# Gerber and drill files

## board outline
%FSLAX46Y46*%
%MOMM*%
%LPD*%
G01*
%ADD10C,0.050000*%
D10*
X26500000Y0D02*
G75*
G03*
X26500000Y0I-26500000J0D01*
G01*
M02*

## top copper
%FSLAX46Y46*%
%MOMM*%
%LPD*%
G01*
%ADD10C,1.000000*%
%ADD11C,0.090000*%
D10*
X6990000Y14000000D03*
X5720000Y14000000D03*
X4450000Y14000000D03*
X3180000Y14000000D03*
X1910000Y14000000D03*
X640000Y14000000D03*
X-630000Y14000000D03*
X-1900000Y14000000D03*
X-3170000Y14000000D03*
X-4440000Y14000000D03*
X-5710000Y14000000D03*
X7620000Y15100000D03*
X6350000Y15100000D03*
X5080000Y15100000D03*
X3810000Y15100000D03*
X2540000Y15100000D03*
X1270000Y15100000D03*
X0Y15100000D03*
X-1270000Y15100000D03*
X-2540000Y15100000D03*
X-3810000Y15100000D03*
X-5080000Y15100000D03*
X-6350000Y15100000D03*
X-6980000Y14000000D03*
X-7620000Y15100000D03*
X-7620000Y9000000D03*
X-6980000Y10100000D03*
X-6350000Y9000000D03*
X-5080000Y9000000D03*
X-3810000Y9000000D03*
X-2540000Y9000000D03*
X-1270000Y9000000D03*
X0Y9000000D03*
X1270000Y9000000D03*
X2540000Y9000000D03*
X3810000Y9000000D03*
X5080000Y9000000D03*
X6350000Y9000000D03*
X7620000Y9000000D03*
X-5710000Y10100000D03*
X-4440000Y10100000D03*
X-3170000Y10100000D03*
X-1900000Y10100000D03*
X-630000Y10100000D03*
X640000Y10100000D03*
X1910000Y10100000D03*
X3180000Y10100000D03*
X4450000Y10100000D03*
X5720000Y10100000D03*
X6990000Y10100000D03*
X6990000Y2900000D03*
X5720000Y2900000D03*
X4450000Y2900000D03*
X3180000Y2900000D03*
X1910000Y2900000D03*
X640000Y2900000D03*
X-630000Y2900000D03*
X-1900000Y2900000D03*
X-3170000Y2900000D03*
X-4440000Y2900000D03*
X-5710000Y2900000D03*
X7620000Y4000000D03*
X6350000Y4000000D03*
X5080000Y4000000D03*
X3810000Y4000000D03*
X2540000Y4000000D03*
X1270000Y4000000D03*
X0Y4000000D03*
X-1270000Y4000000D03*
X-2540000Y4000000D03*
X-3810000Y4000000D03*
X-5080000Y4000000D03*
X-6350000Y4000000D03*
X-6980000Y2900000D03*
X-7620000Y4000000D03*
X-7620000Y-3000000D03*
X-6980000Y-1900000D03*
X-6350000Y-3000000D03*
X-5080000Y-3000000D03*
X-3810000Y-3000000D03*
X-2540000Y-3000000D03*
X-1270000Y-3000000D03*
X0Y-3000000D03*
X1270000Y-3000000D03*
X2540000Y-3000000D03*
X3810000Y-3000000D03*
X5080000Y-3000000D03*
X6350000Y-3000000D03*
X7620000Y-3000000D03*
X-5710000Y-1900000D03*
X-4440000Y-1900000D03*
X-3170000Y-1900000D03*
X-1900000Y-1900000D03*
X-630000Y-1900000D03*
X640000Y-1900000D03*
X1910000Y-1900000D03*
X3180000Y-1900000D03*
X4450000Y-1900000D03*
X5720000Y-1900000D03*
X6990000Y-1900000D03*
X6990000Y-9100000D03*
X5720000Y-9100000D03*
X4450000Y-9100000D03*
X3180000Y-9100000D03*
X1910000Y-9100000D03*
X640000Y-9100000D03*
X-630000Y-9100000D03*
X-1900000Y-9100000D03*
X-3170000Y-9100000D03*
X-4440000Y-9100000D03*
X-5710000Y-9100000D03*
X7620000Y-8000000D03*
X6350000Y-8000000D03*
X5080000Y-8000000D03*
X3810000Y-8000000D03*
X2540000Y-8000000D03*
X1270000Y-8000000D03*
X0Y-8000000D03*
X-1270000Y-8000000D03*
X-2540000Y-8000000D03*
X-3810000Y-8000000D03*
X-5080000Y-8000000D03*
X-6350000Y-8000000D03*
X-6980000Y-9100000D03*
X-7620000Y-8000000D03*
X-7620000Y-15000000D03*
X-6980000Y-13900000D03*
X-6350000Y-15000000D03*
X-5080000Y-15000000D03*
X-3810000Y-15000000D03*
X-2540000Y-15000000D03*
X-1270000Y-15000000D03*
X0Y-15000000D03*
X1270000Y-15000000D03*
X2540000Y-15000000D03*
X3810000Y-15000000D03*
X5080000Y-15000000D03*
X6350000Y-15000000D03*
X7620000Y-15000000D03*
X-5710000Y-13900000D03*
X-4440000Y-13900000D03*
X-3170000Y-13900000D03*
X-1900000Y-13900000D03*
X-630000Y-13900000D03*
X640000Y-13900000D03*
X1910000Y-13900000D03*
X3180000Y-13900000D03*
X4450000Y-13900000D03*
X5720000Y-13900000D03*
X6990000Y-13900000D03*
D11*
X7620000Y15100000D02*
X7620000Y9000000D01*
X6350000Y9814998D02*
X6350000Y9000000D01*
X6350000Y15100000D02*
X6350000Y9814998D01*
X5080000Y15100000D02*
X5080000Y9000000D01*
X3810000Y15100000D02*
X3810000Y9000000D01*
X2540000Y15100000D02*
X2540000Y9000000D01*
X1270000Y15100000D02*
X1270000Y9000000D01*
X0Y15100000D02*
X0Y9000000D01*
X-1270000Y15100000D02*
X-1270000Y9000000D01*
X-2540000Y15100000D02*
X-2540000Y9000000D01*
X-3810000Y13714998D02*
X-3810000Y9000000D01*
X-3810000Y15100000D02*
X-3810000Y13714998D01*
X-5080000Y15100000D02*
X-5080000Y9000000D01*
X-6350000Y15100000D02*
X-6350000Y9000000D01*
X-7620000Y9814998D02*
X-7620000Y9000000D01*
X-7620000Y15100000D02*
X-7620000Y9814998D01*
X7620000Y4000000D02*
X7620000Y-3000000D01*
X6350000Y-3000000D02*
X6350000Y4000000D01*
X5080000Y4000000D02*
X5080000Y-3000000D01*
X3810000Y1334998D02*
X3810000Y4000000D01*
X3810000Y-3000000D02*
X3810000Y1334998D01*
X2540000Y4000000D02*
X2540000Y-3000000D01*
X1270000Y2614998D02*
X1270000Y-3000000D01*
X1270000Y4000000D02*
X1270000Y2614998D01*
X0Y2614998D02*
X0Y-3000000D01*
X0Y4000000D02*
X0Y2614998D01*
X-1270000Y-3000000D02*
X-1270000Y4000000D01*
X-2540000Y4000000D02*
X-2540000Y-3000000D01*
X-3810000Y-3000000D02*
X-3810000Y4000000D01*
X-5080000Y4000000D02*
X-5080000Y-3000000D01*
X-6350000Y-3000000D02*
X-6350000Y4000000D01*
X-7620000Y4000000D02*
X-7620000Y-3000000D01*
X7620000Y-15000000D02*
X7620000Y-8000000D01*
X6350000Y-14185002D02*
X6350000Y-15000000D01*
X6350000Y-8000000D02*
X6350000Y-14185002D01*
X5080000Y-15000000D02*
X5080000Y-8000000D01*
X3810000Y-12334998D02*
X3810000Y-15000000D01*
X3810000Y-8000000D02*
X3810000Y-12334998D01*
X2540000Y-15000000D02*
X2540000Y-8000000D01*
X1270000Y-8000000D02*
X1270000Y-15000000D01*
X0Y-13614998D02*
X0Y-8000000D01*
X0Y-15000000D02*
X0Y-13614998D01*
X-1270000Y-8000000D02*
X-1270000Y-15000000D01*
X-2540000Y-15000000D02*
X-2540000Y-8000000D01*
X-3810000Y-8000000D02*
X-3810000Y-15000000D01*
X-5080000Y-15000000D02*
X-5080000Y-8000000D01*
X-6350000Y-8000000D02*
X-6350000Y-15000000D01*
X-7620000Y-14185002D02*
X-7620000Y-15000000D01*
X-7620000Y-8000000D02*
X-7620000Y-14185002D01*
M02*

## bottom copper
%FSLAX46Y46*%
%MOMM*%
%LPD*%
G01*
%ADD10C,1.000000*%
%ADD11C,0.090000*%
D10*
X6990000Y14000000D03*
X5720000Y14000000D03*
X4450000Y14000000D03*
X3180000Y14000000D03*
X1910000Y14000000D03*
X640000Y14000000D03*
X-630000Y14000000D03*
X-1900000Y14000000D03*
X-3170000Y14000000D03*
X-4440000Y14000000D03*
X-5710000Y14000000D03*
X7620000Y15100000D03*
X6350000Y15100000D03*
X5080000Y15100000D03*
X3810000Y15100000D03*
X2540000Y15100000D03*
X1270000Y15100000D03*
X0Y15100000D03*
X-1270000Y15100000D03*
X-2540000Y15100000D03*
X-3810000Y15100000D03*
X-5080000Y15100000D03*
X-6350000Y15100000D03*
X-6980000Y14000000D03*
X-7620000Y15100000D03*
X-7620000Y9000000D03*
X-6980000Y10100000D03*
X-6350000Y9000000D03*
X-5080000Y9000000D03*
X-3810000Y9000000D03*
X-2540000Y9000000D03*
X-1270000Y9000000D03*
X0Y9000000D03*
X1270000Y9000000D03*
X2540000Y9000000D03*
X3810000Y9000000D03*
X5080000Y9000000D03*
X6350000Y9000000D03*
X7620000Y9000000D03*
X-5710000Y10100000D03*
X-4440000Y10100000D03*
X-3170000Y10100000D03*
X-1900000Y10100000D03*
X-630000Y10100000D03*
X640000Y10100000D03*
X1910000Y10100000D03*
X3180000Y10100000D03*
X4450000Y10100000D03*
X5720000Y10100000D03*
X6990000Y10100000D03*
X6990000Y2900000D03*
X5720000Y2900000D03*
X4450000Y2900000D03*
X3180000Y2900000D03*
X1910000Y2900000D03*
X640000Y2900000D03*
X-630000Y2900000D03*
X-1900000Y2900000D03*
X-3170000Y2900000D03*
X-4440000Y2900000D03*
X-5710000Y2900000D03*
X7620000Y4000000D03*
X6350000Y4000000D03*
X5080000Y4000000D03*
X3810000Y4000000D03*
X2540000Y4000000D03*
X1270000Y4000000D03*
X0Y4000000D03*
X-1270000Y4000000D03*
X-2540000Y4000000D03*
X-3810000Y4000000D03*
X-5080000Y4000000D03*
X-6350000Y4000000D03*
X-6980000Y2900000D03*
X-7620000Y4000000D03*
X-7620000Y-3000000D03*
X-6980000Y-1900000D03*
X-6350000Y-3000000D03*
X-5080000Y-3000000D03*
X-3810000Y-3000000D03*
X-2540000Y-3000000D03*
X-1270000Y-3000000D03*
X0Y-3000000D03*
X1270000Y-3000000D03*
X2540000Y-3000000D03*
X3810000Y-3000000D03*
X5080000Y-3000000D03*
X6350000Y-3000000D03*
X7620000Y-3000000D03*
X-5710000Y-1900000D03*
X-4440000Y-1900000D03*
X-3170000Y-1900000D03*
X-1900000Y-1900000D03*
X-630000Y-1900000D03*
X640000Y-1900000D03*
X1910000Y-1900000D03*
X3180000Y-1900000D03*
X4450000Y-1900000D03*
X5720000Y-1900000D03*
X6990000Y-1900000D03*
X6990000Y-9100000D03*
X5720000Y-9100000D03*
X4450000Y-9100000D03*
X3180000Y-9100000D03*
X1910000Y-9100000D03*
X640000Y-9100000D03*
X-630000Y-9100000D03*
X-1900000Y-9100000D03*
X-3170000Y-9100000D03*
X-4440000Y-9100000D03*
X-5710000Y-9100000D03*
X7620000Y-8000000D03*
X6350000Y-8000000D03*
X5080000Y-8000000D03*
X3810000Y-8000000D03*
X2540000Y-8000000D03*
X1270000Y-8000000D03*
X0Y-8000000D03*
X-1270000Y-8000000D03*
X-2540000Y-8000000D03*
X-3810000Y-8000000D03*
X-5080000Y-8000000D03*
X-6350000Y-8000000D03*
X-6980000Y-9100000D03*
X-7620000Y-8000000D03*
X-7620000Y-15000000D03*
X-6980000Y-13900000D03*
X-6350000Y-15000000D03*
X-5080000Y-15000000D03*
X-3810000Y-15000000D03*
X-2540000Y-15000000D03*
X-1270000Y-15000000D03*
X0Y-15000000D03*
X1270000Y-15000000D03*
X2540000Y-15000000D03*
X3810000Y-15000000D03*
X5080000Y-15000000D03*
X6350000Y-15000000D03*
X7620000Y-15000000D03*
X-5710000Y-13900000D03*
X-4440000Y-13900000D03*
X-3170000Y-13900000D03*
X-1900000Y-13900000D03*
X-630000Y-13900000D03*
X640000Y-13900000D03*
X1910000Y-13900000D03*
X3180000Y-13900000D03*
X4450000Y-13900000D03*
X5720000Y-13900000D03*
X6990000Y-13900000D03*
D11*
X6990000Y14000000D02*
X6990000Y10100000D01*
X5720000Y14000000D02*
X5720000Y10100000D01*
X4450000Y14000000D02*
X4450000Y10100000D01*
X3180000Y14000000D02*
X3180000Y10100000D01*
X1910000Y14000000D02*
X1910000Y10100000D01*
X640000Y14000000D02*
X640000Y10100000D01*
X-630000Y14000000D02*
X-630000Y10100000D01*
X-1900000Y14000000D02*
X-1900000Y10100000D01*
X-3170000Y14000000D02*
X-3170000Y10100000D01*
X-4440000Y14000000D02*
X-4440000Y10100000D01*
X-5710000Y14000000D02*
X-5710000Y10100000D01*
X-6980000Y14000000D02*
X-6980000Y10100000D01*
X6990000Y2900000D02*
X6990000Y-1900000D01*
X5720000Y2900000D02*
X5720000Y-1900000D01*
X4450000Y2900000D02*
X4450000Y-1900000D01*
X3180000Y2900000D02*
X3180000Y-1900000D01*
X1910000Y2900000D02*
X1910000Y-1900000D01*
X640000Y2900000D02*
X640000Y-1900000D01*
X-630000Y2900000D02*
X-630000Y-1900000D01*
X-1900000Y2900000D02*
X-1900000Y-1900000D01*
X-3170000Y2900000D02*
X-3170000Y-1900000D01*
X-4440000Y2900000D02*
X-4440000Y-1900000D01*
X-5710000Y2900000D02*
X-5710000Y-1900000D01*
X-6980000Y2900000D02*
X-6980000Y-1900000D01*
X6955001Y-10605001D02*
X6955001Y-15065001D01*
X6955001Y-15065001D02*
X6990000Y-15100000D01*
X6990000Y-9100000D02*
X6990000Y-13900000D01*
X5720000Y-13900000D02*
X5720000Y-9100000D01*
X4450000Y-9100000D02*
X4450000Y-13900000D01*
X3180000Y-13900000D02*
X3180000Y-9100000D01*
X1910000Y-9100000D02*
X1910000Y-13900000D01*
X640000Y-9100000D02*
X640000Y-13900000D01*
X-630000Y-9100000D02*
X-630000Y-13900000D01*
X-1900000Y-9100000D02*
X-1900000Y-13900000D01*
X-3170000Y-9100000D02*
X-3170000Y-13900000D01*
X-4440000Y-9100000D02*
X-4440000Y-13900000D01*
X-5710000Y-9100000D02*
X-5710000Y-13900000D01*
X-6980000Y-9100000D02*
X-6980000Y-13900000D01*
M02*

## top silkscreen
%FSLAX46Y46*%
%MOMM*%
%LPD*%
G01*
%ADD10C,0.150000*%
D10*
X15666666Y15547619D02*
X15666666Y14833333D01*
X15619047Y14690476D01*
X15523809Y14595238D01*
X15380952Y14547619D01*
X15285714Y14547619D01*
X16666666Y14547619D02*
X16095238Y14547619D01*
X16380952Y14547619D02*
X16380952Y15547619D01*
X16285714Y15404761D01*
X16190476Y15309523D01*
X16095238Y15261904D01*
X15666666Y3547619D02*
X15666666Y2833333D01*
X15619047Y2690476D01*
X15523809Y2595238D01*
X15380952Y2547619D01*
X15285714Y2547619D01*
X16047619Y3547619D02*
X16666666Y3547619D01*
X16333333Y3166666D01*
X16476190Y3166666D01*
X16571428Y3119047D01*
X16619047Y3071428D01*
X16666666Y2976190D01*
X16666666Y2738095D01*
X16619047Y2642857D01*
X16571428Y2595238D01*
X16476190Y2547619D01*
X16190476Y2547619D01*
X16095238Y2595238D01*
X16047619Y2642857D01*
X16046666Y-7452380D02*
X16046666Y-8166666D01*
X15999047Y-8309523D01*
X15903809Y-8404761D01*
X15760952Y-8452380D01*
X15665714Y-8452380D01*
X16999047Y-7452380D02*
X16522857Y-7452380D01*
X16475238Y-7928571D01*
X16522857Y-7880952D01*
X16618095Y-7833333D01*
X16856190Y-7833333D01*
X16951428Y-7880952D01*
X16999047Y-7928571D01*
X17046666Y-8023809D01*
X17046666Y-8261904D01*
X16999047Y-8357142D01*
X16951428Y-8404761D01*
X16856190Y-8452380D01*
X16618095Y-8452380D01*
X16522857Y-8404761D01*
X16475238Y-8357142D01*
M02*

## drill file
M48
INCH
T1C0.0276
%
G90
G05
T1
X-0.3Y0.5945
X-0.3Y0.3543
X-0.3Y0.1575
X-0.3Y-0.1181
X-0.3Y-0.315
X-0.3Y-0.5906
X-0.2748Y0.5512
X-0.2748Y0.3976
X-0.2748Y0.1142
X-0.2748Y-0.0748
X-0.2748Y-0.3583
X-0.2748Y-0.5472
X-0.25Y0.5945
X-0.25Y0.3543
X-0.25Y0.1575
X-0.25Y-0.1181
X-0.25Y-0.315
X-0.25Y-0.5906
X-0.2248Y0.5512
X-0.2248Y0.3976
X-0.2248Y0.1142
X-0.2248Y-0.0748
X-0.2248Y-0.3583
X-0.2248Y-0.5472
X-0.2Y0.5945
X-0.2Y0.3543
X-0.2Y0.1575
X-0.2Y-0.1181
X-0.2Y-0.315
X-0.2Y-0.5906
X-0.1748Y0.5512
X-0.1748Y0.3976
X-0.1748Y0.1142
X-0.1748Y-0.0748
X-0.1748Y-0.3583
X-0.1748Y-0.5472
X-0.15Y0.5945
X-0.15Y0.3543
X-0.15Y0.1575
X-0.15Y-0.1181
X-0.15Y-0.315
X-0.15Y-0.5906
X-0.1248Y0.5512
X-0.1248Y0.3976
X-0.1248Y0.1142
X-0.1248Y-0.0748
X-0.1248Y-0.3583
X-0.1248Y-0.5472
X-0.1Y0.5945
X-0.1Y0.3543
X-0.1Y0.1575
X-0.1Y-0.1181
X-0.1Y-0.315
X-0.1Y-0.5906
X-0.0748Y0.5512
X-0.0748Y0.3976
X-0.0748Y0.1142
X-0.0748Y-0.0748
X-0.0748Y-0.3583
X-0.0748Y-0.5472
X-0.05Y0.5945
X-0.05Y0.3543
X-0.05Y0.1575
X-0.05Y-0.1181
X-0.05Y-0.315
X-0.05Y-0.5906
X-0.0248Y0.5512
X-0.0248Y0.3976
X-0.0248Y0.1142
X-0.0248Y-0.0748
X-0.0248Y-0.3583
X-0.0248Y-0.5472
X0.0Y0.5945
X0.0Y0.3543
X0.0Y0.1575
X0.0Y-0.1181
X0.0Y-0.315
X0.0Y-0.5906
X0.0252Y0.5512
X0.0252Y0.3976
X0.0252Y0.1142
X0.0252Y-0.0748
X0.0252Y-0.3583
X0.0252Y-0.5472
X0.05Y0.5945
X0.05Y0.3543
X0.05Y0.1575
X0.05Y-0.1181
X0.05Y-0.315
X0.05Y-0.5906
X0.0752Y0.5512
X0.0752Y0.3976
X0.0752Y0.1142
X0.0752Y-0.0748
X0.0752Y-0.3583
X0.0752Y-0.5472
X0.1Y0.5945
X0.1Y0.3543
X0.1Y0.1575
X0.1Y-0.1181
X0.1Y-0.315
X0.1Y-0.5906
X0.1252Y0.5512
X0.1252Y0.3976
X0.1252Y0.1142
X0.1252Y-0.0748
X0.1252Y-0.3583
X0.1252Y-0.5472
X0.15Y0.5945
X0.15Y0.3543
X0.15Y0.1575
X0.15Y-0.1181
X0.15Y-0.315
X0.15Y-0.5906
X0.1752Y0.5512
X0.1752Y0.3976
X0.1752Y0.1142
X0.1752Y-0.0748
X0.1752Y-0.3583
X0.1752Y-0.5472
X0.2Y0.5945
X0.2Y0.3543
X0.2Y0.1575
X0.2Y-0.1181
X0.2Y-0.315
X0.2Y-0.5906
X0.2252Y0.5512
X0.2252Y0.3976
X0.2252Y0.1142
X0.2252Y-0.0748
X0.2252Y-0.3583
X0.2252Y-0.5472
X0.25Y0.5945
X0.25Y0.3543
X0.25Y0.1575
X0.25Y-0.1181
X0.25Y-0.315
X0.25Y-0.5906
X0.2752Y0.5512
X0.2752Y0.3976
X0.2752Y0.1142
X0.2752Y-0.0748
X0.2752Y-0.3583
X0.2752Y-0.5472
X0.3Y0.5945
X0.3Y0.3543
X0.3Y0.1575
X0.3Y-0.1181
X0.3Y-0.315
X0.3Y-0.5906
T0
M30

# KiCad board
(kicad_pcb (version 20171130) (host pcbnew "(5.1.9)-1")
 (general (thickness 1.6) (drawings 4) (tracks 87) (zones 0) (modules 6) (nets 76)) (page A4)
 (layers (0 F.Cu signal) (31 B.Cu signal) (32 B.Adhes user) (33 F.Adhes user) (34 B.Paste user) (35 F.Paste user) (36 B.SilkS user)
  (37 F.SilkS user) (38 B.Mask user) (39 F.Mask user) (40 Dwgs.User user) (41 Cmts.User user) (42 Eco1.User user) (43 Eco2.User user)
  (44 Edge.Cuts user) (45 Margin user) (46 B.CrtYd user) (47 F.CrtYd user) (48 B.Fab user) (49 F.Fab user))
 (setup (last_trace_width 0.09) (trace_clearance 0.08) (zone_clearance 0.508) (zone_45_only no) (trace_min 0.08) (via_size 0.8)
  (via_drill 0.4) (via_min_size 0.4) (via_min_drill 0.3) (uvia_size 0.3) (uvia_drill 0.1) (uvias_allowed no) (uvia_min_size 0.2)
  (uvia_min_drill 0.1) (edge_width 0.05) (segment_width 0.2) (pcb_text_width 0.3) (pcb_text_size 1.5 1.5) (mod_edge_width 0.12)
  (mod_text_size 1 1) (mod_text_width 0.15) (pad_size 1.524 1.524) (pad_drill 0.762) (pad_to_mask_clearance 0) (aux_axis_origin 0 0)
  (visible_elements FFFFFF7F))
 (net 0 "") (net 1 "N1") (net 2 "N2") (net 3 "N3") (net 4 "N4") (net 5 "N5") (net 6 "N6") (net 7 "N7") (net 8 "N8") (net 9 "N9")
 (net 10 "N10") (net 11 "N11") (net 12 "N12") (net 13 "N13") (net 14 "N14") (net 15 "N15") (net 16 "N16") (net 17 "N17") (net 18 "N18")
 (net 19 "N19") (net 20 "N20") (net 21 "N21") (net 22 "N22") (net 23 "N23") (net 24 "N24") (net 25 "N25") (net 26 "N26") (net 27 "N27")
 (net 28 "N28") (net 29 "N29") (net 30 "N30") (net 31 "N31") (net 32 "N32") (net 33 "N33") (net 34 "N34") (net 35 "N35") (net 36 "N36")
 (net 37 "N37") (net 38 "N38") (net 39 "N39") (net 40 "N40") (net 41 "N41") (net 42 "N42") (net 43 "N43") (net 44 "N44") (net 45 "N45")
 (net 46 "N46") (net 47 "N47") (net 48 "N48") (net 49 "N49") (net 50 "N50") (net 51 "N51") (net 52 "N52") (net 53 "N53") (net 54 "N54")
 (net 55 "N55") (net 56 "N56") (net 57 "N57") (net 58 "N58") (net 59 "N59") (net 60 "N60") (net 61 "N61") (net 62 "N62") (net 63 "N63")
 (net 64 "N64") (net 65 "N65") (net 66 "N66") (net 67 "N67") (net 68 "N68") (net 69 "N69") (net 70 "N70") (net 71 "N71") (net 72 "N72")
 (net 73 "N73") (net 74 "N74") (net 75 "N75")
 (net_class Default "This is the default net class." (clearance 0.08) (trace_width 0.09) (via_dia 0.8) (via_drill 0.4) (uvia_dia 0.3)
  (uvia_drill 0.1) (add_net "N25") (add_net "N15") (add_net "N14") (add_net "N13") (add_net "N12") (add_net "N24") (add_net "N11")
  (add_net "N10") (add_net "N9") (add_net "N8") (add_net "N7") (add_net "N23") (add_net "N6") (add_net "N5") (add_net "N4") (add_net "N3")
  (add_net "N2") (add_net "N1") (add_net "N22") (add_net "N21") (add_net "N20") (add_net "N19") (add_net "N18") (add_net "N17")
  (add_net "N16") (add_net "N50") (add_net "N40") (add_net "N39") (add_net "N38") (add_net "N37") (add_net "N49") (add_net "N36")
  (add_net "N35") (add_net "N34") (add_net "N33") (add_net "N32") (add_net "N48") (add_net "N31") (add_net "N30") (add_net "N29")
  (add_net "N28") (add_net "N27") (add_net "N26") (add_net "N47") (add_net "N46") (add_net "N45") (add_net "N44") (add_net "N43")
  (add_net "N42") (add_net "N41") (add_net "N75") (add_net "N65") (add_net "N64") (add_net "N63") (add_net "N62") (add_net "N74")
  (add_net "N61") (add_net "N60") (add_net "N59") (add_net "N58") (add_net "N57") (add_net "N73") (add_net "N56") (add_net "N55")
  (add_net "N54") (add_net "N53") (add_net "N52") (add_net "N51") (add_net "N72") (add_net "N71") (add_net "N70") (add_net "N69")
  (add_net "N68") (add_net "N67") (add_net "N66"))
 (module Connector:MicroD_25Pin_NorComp (layer F.Cu) (at -7.62 -15.1)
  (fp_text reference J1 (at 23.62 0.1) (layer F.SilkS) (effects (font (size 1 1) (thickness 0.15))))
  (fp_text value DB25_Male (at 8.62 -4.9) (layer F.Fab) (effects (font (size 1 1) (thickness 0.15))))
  (pad 25 thru_hole circle (at 14.61 1.1) (size 1 1) (drill 0.7) (layers *.Cu *.Mask) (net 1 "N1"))
  (pad 24 thru_hole circle (at 13.34 1.1) (size 1 1) (drill 0.7) (layers *.Cu *.Mask) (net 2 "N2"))
  (pad 23 thru_hole circle (at 12.07 1.1) (size 1 1) (drill 0.7) (layers *.Cu *.Mask) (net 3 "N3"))
  (pad 22 thru_hole circle (at 10.8 1.1) (size 1 1) (drill 0.7) (layers *.Cu *.Mask) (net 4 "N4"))
  (pad 21 thru_hole circle (at 9.53 1.1) (size 1 1) (drill 0.7) (layers *.Cu *.Mask) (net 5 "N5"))
  (pad 20 thru_hole circle (at 8.26 1.1) (size 1 1) (drill 0.7) (layers *.Cu *.Mask) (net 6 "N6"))
  (pad 19 thru_hole circle (at 6.99 1.1) (size 1 1) (drill 0.7) (layers *.Cu *.Mask) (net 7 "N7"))
  (pad 18 thru_hole circle (at 5.72 1.1) (size 1 1) (drill 0.7) (layers *.Cu *.Mask) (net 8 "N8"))
  (pad 17 thru_hole circle (at 4.45 1.1) (size 1 1) (drill 0.7) (layers *.Cu *.Mask) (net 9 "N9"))
  (pad 16 thru_hole circle (at 3.18 1.1) (size 1 1) (drill 0.7) (layers *.Cu *.Mask) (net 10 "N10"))
  (pad 15 thru_hole circle (at 1.91 1.1) (size 1 1) (drill 0.7) (layers *.Cu *.Mask) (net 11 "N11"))
  (pad 13 thru_hole circle (at 15.24 0) (size 1 1) (drill 0.7) (layers *.Cu *.Mask) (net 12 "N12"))
  (pad 12 thru_hole circle (at 13.97 0) (size 1 1) (drill 0.7) (layers *.Cu *.Mask) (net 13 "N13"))
  (pad 11 thru_hole circle (at 12.7 0) (size 1 1) (drill 0.7) (layers *.Cu *.Mask) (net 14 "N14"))
  (pad 10 thru_hole circle (at 11.43 0) (size 1 1) (drill 0.7) (layers *.Cu *.Mask) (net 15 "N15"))
  (pad 9 thru_hole circle (at 10.16 0) (size 1 1) (drill 0.7) (layers *.Cu *.Mask) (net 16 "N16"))
  (pad 8 thru_hole circle (at 8.89 0) (size 1 1) (drill 0.7) (layers *.Cu *.Mask) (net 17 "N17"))
  (pad 7 thru_hole circle (at 7.62 0) (size 1 1) (drill 0.7) (layers *.Cu *.Mask) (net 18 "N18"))
  (pad 6 thru_hole circle (at 6.35 0) (size 1 1) (drill 0.7) (layers *.Cu *.Mask) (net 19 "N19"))
  (pad 5 thru_hole circle (at 5.08 0) (size 1 1) (drill 0.7) (layers *.Cu *.Mask) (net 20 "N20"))
  (pad 4 thru_hole circle (at 3.81 0) (size 1 1) (drill 0.7) (layers *.Cu *.Mask) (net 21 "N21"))
  (pad 3 thru_hole circle (at 2.54 0) (size 1 1) (drill 0.7) (layers *.Cu *.Mask) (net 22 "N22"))
  (pad 2 thru_hole circle (at 1.27 0) (size 1 1) (drill 0.7) (layers *.Cu *.Mask) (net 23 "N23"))
  (pad 14 thru_hole circle (at 0.64 1.1) (size 1 1) (drill 0.7) (layers *.Cu *.Mask) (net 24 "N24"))
  (pad 1 thru_hole circle (at 0 0) (size 1 1) (drill 0.7) (layers *.Cu *.Mask) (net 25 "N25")))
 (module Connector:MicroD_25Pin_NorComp (layer B.Cu) (at -7.62 -9)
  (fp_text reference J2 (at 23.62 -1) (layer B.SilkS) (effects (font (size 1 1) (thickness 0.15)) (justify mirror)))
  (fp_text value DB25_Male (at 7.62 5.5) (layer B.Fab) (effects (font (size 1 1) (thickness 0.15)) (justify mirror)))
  (pad 1 thru_hole circle (at 0 0) (size 1 1) (drill 0.7) (layers *.Cu *.Mask) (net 25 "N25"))
  (pad 14 thru_hole circle (at 0.64 -1.1) (size 1 1) (drill 0.7) (layers *.Cu *.Mask) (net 24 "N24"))
  (pad 2 thru_hole circle (at 1.27 0) (size 1 1) (drill 0.7) (layers *.Cu *.Mask) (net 23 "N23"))
  (pad 3 thru_hole circle (at 2.54 0) (size 1 1) (drill 0.7) (layers *.Cu *.Mask) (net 22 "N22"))
  (pad 4 thru_hole circle (at 3.81 0) (size 1 1) (drill 0.7) (layers *.Cu *.Mask) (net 21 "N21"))
  (pad 5 thru_hole circle (at 5.08 0) (size 1 1) (drill 0.7) (layers *.Cu *.Mask) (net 20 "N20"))
  (pad 6 thru_hole circle (at 6.35 0) (size 1 1) (drill 0.7) (layers *.Cu *.Mask) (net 19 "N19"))
  (pad 7 thru_hole circle (at 7.62 0) (size 1 1) (drill 0.7) (layers *.Cu *.Mask) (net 18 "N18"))
  (pad 8 thru_hole circle (at 8.89 0) (size 1 1) (drill 0.7) (layers *.Cu *.Mask) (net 17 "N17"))
  (pad 9 thru_hole circle (at 10.16 0) (size 1 1) (drill 0.7) (layers *.Cu *.Mask) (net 16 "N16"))
  (pad 10 thru_hole circle (at 11.43 0) (size 1 1) (drill 0.7) (layers *.Cu *.Mask) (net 15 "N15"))
  (pad 11 thru_hole circle (at 12.7 0) (size 1 1) (drill 0.7) (layers *.Cu *.Mask) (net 14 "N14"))
  (pad 12 thru_hole circle (at 13.97 0) (size 1 1) (drill 0.7) (layers *.Cu *.Mask) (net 13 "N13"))
  (pad 13 thru_hole circle (at 15.24 0) (size 1 1) (drill 0.7) (layers *.Cu *.Mask) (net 12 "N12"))
  (pad 15 thru_hole circle (at 1.91 -1.1) (size 1 1) (drill 0.7) (layers *.Cu *.Mask) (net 11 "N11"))
  (pad 16 thru_hole circle (at 3.18 -1.1) (size 1 1) (drill 0.7) (layers *.Cu *.Mask) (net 10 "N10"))
  (pad 17 thru_hole circle (at 4.45 -1.1) (size 1 1) (drill 0.7) (layers *.Cu *.Mask) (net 9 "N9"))
  (pad 18 thru_hole circle (at 5.72 -1.1) (size 1 1) (drill 0.7) (layers *.Cu *.Mask) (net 8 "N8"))
  (pad 19 thru_hole circle (at 6.99 -1.1) (size 1 1) (drill 0.7) (layers *.Cu *.Mask) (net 7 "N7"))
  (pad 20 thru_hole circle (at 8.26 -1.1) (size 1 1) (drill 0.7) (layers *.Cu *.Mask) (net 6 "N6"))
  (pad 21 thru_hole circle (at 9.53 -1.1) (size 1 1) (drill 0.7) (layers *.Cu *.Mask) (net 5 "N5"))
  (pad 22 thru_hole circle (at 10.8 -1.1) (size 1 1) (drill 0.7) (layers *.Cu *.Mask) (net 4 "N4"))
  (pad 23 thru_hole circle (at 12.07 -1.1) (size 1 1) (drill 0.7) (layers *.Cu *.Mask) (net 3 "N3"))
  (pad 24 thru_hole circle (at 13.34 -1.1) (size 1 1) (drill 0.7) (layers *.Cu *.Mask) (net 2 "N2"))
  (pad 25 thru_hole circle (at 14.61 -1.1) (size 1 1) (drill 0.7) (layers *.Cu *.Mask) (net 1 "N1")))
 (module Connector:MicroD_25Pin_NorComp (layer F.Cu) (at -7.62 -4)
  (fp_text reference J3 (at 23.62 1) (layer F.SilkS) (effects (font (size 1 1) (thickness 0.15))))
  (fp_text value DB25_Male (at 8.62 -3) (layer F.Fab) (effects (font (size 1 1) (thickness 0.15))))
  (pad 25 thru_hole circle (at 14.61 1.1) (size 1 1) (drill 0.7) (layers *.Cu *.Mask) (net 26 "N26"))
  (pad 24 thru_hole circle (at 13.34 1.1) (size 1 1) (drill 0.7) (layers *.Cu *.Mask) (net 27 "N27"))
  (pad 23 thru_hole circle (at 12.07 1.1) (size 1 1) (drill 0.7) (layers *.Cu *.Mask) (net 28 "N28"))
  (pad 22 thru_hole circle (at 10.8 1.1) (size 1 1) (drill 0.7) (layers *.Cu *.Mask) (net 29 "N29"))
  (pad 21 thru_hole circle (at 9.53 1.1) (size 1 1) (drill 0.7) (layers *.Cu *.Mask) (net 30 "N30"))
  (pad 20 thru_hole circle (at 8.26 1.1) (size 1 1) (drill 0.7) (layers *.Cu *.Mask) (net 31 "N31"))
  (pad 19 thru_hole circle (at 6.99 1.1) (size 1 1) (drill 0.7) (layers *.Cu *.Mask) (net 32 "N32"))
  (pad 18 thru_hole circle (at 5.72 1.1) (size 1 1) (drill 0.7) (layers *.Cu *.Mask) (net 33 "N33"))
  (pad 17 thru_hole circle (at 4.45 1.1) (size 1 1) (drill 0.7) (layers *.Cu *.Mask) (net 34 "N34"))
  (pad 16 thru_hole circle (at 3.18 1.1) (size 1 1) (drill 0.7) (layers *.Cu *.Mask) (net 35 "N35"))
  (pad 15 thru_hole circle (at 1.91 1.1) (size 1 1) (drill 0.7) (layers *.Cu *.Mask) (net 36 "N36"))
  (pad 13 thru_hole circle (at 15.24 0) (size 1 1) (drill 0.7) (layers *.Cu *.Mask) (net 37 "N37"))
  (pad 12 thru_hole circle (at 13.97 0) (size 1 1) (drill 0.7) (layers *.Cu *.Mask) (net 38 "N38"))
  (pad 11 thru_hole circle (at 12.7 0) (size 1 1) (drill 0.7) (layers *.Cu *.Mask) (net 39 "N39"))
  (pad 10 thru_hole circle (at 11.43 0) (size 1 1) (drill 0.7) (layers *.Cu *.Mask) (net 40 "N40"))
  (pad 9 thru_hole circle (at 10.16 0) (size 1 1) (drill 0.7) (layers *.Cu *.Mask) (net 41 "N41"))
  (pad 8 thru_hole circle (at 8.89 0) (size 1 1) (drill 0.7) (layers *.Cu *.Mask) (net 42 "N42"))
  (pad 7 thru_hole circle (at 7.62 0) (size 1 1) (drill 0.7) (layers *.Cu *.Mask) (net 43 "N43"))
  (pad 6 thru_hole circle (at 6.35 0) (size 1 1) (drill 0.7) (layers *.Cu *.Mask) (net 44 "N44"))
  (pad 5 thru_hole circle (at 5.08 0) (size 1 1) (drill 0.7) (layers *.Cu *.Mask) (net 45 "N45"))
  (pad 4 thru_hole circle (at 3.81 0) (size 1 1) (drill 0.7) (layers *.Cu *.Mask) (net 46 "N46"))
  (pad 3 thru_hole circle (at 2.54 0) (size 1 1) (drill 0.7) (layers *.Cu *.Mask) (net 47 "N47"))
  (pad 2 thru_hole circle (at 1.27 0) (size 1 1) (drill 0.7) (layers *.Cu *.Mask) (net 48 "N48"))
  (pad 14 thru_hole circle (at 0.64 1.1) (size 1 1) (drill 0.7) (layers *.Cu *.Mask) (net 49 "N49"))
  (pad 1 thru_hole circle (at 0 0) (size 1 1) (drill 0.7) (layers *.Cu *.Mask) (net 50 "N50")))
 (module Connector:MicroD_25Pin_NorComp (layer B.Cu) (at -7.62 3)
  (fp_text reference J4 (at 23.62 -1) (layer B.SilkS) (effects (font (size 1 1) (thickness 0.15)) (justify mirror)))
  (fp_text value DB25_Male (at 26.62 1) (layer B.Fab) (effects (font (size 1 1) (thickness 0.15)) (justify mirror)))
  (pad 1 thru_hole circle (at 0 0) (size 1 1) (drill 0.7) (layers *.Cu *.Mask) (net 50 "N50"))
  (pad 14 thru_hole circle (at 0.64 -1.1) (size 1 1) (drill 0.7) (layers *.Cu *.Mask) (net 49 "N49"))
  (pad 2 thru_hole circle (at 1.27 0) (size 1 1) (drill 0.7) (layers *.Cu *.Mask) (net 48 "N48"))
  (pad 3 thru_hole circle (at 2.54 0) (size 1 1) (drill 0.7) (layers *.Cu *.Mask) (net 47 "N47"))
  (pad 4 thru_hole circle (at 3.81 0) (size 1 1) (drill 0.7) (layers *.Cu *.Mask) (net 46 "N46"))
  (pad 5 thru_hole circle (at 5.08 0) (size 1 1) (drill 0.7) (layers *.Cu *.Mask) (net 45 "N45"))
  (pad 6 thru_hole circle (at 6.35 0) (size 1 1) (drill 0.7) (layers *.Cu *.Mask) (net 44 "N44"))
  (pad 7 thru_hole circle (at 7.62 0) (size 1 1) (drill 0.7) (layers *.Cu *.Mask) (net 43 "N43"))
  (pad 8 thru_hole circle (at 8.89 0) (size 1 1) (drill 0.7) (layers *.Cu *.Mask) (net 42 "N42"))
  (pad 9 thru_hole circle (at 10.16 0) (size 1 1) (drill 0.7) (layers *.Cu *.Mask) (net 41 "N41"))
  (pad 10 thru_hole circle (at 11.43 0) (size 1 1) (drill 0.7) (layers *.Cu *.Mask) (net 40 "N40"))
  (pad 11 thru_hole circle (at 12.7 0) (size 1 1) (drill 0.7) (layers *.Cu *.Mask) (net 39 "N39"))
  (pad 12 thru_hole circle (at 13.97 0) (size 1 1) (drill 0.7) (layers *.Cu *.Mask) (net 38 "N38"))
  (pad 13 thru_hole circle (at 15.24 0) (size 1 1) (drill 0.7) (layers *.Cu *.Mask) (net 37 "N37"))
  (pad 15 thru_hole circle (at 1.91 -1.1) (size 1 1) (drill 0.7) (layers *.Cu *.Mask) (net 36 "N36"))
  (pad 16 thru_hole circle (at 3.18 -1.1) (size 1 1) (drill 0.7) (layers *.Cu *.Mask) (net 35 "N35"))
  (pad 17 thru_hole circle (at 4.45 -1.1) (size 1 1) (drill 0.7) (layers *.Cu *.Mask) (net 34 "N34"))
  (pad 18 thru_hole circle (at 5.72 -1.1) (size 1 1) (drill 0.7) (layers *.Cu *.Mask) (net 33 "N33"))
  (pad 19 thru_hole circle (at 6.99 -1.1) (size 1 1) (drill 0.7) (layers *.Cu *.Mask) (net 32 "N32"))
  (pad 20 thru_hole circle (at 8.26 -1.1) (size 1 1) (drill 0.7) (layers *.Cu *.Mask) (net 31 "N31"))
  (pad 21 thru_hole circle (at 9.53 -1.1) (size 1 1) (drill 0.7) (layers *.Cu *.Mask) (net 30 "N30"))
  (pad 22 thru_hole circle (at 10.8 -1.1) (size 1 1) (drill 0.7) (layers *.Cu *.Mask) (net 29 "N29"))
  (pad 23 thru_hole circle (at 12.07 -1.1) (size 1 1) (drill 0.7) (layers *.Cu *.Mask) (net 28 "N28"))
  (pad 24 thru_hole circle (at 13.34 -1.1) (size 1 1) (drill 0.7) (layers *.Cu *.Mask) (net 27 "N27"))
  (pad 25 thru_hole circle (at 14.61 -1.1) (size 1 1) (drill 0.7) (layers *.Cu *.Mask) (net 26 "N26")))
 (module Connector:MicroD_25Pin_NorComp (layer F.Cu) (at -7.62 8)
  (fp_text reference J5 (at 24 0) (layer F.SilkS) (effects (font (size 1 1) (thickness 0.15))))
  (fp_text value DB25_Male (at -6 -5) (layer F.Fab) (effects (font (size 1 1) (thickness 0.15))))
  (pad 25 thru_hole circle (at 14.61 1.1) (size 1 1) (drill 0.7) (layers *.Cu *.Mask) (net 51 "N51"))
  (pad 24 thru_hole circle (at 13.34 1.1) (size 1 1) (drill 0.7) (layers *.Cu *.Mask) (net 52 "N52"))
  (pad 23 thru_hole circle (at 12.07 1.1) (size 1 1) (drill 0.7) (layers *.Cu *.Mask) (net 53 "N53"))
  (pad 22 thru_hole circle (at 10.8 1.1) (size 1 1) (drill 0.7) (layers *.Cu *.Mask) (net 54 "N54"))
  (pad 21 thru_hole circle (at 9.53 1.1) (size 1 1) (drill 0.7) (layers *.Cu *.Mask) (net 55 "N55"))
  (pad 20 thru_hole circle (at 8.26 1.1) (size 1 1) (drill 0.7) (layers *.Cu *.Mask) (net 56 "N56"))
  (pad 19 thru_hole circle (at 6.99 1.1) (size 1 1) (drill 0.7) (layers *.Cu *.Mask) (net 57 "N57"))
  (pad 18 thru_hole circle (at 5.72 1.1) (size 1 1) (drill 0.7) (layers *.Cu *.Mask) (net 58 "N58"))
  (pad 17 thru_hole circle (at 4.45 1.1) (size 1 1) (drill 0.7) (layers *.Cu *.Mask) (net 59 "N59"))
  (pad 16 thru_hole circle (at 3.18 1.1) (size 1 1) (drill 0.7) (layers *.Cu *.Mask) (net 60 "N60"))
  (pad 15 thru_hole circle (at 1.91 1.1) (size 1 1) (drill 0.7) (layers *.Cu *.Mask) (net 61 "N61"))
  (pad 13 thru_hole circle (at 15.24 0) (size 1 1) (drill 0.7) (layers *.Cu *.Mask) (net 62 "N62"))
  (pad 12 thru_hole circle (at 13.97 0) (size 1 1) (drill 0.7) (layers *.Cu *.Mask) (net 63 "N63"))
  (pad 11 thru_hole circle (at 12.7 0) (size 1 1) (drill 0.7) (layers *.Cu *.Mask) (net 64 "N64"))
  (pad 10 thru_hole circle (at 11.43 0) (size 1 1) (drill 0.7) (layers *.Cu *.Mask) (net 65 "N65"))
  (pad 9 thru_hole circle (at 10.16 0) (size 1 1) (drill 0.7) (layers *.Cu *.Mask) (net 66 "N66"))
  (pad 8 thru_hole circle (at 8.89 0) (size 1 1) (drill 0.7) (layers *.Cu *.Mask) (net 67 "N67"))
  (pad 7 thru_hole circle (at 7.62 0) (size 1 1) (drill 0.7) (layers *.Cu *.Mask) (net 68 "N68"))
  (pad 6 thru_hole circle (at 6.35 0) (size 1 1) (drill 0.7) (layers *.Cu *.Mask) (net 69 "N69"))
  (pad 5 thru_hole circle (at 5.08 0) (size 1 1) (drill 0.7) (layers *.Cu *.Mask) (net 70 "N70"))
  (pad 4 thru_hole circle (at 3.81 0) (size 1 1) (drill 0.7) (layers *.Cu *.Mask) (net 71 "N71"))
  (pad 3 thru_hole circle (at 2.54 0) (size 1 1) (drill 0.7) (layers *.Cu *.Mask) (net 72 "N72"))
  (pad 2 thru_hole circle (at 1.27 0) (size 1 1) (drill 0.7) (layers *.Cu *.Mask) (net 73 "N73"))
  (pad 14 thru_hole circle (at 0.64 1.1) (size 1 1) (drill 0.7) (layers *.Cu *.Mask) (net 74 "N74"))
  (pad 1 thru_hole circle (at 0 0) (size 1 1) (drill 0.7) (layers *.Cu *.Mask) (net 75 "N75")))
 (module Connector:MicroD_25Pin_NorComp (layer B.Cu) (at -7.62 15)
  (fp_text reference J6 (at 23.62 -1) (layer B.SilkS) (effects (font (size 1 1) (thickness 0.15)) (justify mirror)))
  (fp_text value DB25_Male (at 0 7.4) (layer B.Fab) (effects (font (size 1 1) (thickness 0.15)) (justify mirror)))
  (pad 1 thru_hole circle (at 0 0) (size 1 1) (drill 0.7) (layers *.Cu *.Mask) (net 75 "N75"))
  (pad 14 thru_hole circle (at 0.64 -1.1) (size 1 1) (drill 0.7) (layers *.Cu *.Mask) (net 74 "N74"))
  (pad 2 thru_hole circle (at 1.27 0) (size 1 1) (drill 0.7) (layers *.Cu *.Mask) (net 73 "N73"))
  (pad 3 thru_hole circle (at 2.54 0) (size 1 1) (drill 0.7) (layers *.Cu *.Mask) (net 72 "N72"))
  (pad 4 thru_hole circle (at 3.81 0) (size 1 1) (drill 0.7) (layers *.Cu *.Mask) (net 71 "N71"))
  (pad 5 thru_hole circle (at 5.08 0) (size 1 1) (drill 0.7) (layers *.Cu *.Mask) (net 70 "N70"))
  (pad 6 thru_hole circle (at 6.35 0) (size 1 1) (drill 0.7) (layers *.Cu *.Mask) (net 69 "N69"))
  (pad 7 thru_hole circle (at 7.62 0) (size 1 1) (drill 0.7) (layers *.Cu *.Mask) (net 68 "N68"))
  (pad 8 thru_hole circle (at 8.89 0) (size 1 1) (drill 0.7) (layers *.Cu *.Mask) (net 67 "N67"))
  (pad 9 thru_hole circle (at 10.16 0) (size 1 1) (drill 0.7) (layers *.Cu *.Mask) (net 66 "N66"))
  (pad 10 thru_hole circle (at 11.43 0) (size 1 1) (drill 0.7) (layers *.Cu *.Mask) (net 65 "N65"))
  (pad 11 thru_hole circle (at 12.7 0) (size 1 1) (drill 0.7) (layers *.Cu *.Mask) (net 64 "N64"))
  (pad 12 thru_hole circle (at 13.97 0) (size 1 1) (drill 0.7) (layers *.Cu *.Mask) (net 63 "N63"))
  (pad 13 thru_hole circle (at 15.24 0) (size 1 1) (drill 0.7) (layers *.Cu *.Mask) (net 62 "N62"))
  (pad 15 thru_hole circle (at 1.91 -1.1) (size 1 1) (drill 0.7) (layers *.Cu *.Mask) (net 61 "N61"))
  (pad 16 thru_hole circle (at 3.18 -1.1) (size 1 1) (drill 0.7) (layers *.Cu *.Mask) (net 60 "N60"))
  (pad 17 thru_hole circle (at 4.45 -1.1) (size 1 1) (drill 0.7) (layers *.Cu *.Mask) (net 59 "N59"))
  (pad 18 thru_hole circle (at 5.72 -1.1) (size 1 1) (drill 0.7) (layers *.Cu *.Mask) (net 58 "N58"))
  (pad 19 thru_hole circle (at 6.99 -1.1) (size 1 1) (drill 0.7) (layers *.Cu *.Mask) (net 57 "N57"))
  (pad 20 thru_hole circle (at 8.26 -1.1) (size 1 1) (drill 0.7) (layers *.Cu *.Mask) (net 56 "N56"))
  (pad 21 thru_hole circle (at 9.53 -1.1) (size 1 1) (drill 0.7) (layers *.Cu *.Mask) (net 55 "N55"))
  (pad 22 thru_hole circle (at 10.8 -1.1) (size 1 1) (drill 0.7) (layers *.Cu *.Mask) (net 54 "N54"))
  (pad 23 thru_hole circle (at 12.07 -1.1) (size 1 1) (drill 0.7) (layers *.Cu *.Mask) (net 53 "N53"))
  (pad 24 thru_hole circle (at 13.34 -1.1) (size 1 1) (drill 0.7) (layers *.Cu *.Mask) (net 52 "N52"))
  (pad 25 thru_hole circle (at 14.61 -1.1) (size 1 1) (drill 0.7) (layers *.Cu *.Mask) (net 51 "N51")))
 (gr_circle (center 0 0) (end 26.5 0) (layer Edge.Cuts) (width 0.05))
 (segment (start 6.99 -14) (end 6.99 -10.1) (width 0.09) (layer B.Cu) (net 1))
 (segment (start 5.72 -14) (end 5.72 -10.1) (width 0.09) (layer B.Cu) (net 2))
 (segment (start 4.45 -14) (end 4.45 -10.1) (width 0.09) (layer B.Cu) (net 3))
 (segment (start 3.18 -14) (end 3.18 -10.1) (width 0.09) (layer B.Cu) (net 4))
 (segment (start 1.91 -14) (end 1.91 -10.1) (width 0.09) (layer B.Cu) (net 5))
 (segment (start 0.64 -14) (end 0.64 -10.1) (width 0.09) (layer B.Cu) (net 6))
 (segment (start -0.63 -14) (end -0.63 -10.1) (width 0.09) (layer B.Cu) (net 7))
 (segment (start -1.9 -14) (end -1.9 -10.1) (width 0.09) (layer B.Cu) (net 8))
 (segment (start -3.17 -14) (end -3.17 -10.1) (width 0.09) (layer B.Cu) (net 9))
 (segment (start -4.44 -14) (end -4.44 -10.1) (width 0.09) (layer B.Cu) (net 10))
 (segment (start -5.71 -14) (end -5.71 -10.1) (width 0.09) (layer B.Cu) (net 11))
 (segment (start 7.62 -15.1) (end 7.62 -9) (width 0.09) (layer F.Cu) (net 12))
 (segment (start 6.35 -9.814998) (end 6.35 -9) (width 0.09) (layer F.Cu) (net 13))
 (segment (start 6.35 -15.1) (end 6.35 -9.814998) (width 0.09) (layer F.Cu) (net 13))
 (segment (start 5.08 -15.1) (end 5.08 -9) (width 0.09) (layer F.Cu) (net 14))
 (segment (start 3.81 -15.1) (end 3.81 -9) (width 0.09) (layer F.Cu) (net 15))
 (segment (start 2.54 -15.1) (end 2.54 -9) (width 0.09) (layer F.Cu) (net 16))
 (segment (start 1.27 -15.1) (end 1.27 -9) (width 0.09) (layer F.Cu) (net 17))
 (segment (start 0 -15.1) (end 0 -9) (width 0.09) (layer F.Cu) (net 18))
 (segment (start -1.27 -15.1) (end -1.27 -9) (width 0.09) (layer F.Cu) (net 19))
 (segment (start -2.54 -15.1) (end -2.54 -9) (width 0.09) (layer F.Cu) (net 20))
 (segment (start -3.81 -13.714998) (end -3.81 -9) (width 0.09) (layer F.Cu) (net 21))
 (segment (start -3.81 -15.1) (end -3.81 -13.714998) (width 0.09) (layer F.Cu) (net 21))
 (segment (start -5.08 -15.1) (end -5.08 -9) (width 0.09) (layer F.Cu) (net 22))
 (segment (start -6.35 -15.1) (end -6.35 -9) (width 0.09) (layer F.Cu) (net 23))
 (segment (start -6.98 -14) (end -6.98 -10.1) (width 0.09) (layer B.Cu) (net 24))
 (segment (start -7.62 -9.814998) (end -7.62 -9) (width 0.09) (layer F.Cu) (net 25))
 (segment (start -7.62 -15.1) (end -7.62 -9.814998) (width 0.09) (layer F.Cu) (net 25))
 (segment (start 6.99 -2.9) (end 6.99 1.9) (width 0.09) (layer B.Cu) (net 26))
 (segment (start 5.72 -2.9) (end 5.72 1.9) (width 0.09) (layer B.Cu) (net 27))
 (segment (start 4.45 -2.9) (end 4.45 1.9) (width 0.09) (layer B.Cu) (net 28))
 (segment (start 3.18 -2.9) (end 3.18 1.9) (width 0.09) (layer B.Cu) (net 29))
 (segment (start 1.91 -2.9) (end 1.91 1.9) (width 0.09) (layer B.Cu) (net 30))
 (segment (start 0.64 -2.9) (end 0.64 1.9) (width 0.09) (layer B.Cu) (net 31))
 (segment (start -0.63 -2.9) (end -0.63 1.9) (width 0.09) (layer B.Cu) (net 32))
 (segment (start -1.9 -2.9) (end -1.9 1.9) (width 0.09) (layer B.Cu) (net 33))
 (segment (start -3.17 -2.9) (end -3.17 1.9) (width 0.09) (layer B.Cu) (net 34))
 (segment (start -4.44 -2.9) (end -4.44 1.9) (width 0.09) (layer B.Cu) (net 35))
 (segment (start -5.71 -2.9) (end -5.71 1.9) (width 0.09) (layer B.Cu) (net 36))
 (segment (start 7.62 -4) (end 7.62 3) (width 0.09) (layer F.Cu) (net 37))
 (segment (start 6.35 3) (end 6.35 -4) (width 0.09) (layer F.Cu) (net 38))
 (segment (start 5.08 -4) (end 5.08 3) (width 0.09) (layer F.Cu) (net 39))
 (segment (start 3.81 -1.334998) (end 3.81 -4) (width 0.09) (layer F.Cu) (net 40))
 (segment (start 3.81 3) (end 3.81 -1.334998) (width 0.09) (layer F.Cu) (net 40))
 (segment (start 2.54 -4) (end 2.54 3) (width 0.09) (layer F.Cu) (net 41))
 (segment (start 1.27 -2.614998) (end 1.27 3) (width 0.09) (layer F.Cu) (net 42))
 (segment (start 1.27 -4) (end 1.27 -2.614998) (width 0.09) (layer F.Cu) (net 42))
 (segment (start 0 -2.614998) (end 0 3) (width 0.09) (layer F.Cu) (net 43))
 (segment (start 0 -4) (end 0 -2.614998) (width 0.09) (layer F.Cu) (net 43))
 (segment (start -1.27 3) (end -1.27 -4) (width 0.09) (layer F.Cu) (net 44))
 (segment (start -2.54 -4) (end -2.54 3) (width 0.09) (layer F.Cu) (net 45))
 (segment (start -3.81 3) (end -3.81 -4) (width 0.09) (layer F.Cu) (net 46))
 (segment (start -5.08 -4) (end -5.08 3) (width 0.09) (layer F.Cu) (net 47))
 (segment (start -6.35 3) (end -6.35 -4) (width 0.09) (layer F.Cu) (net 48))
 (segment (start -6.98 -2.9) (end -6.98 1.9) (width 0.09) (layer B.Cu) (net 49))
 (segment (start -7.62 -4) (end -7.62 3) (width 0.09) (layer F.Cu) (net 50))
 (segment (start 6.955001 10.605001) (end 6.955001 15.065001) (width 0.09) (layer B.Cu) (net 51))
 (segment (start 6.955001 15.065001) (end 6.99 15.1) (width 0.09) (layer B.Cu) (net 51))
 (segment (start 6.99 9.1) (end 6.99 13.9) (width 0.09) (layer B.Cu) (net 51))
 (segment (start 5.72 13.9) (end 5.72 9.1) (width 0.09) (layer B.Cu) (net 52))
 (segment (start 4.45 9.1) (end 4.45 13.9) (width 0.09) (layer B.Cu) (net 53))
 (segment (start 3.18 13.9) (end 3.18 9.1) (width 0.09) (layer B.Cu) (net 54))
 (segment (start 1.91 9.1) (end 1.91 13.9) (width 0.09) (layer B.Cu) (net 55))
 (segment (start 0.64 9.1) (end 0.64 13.9) (width 0.09) (layer B.Cu) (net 56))
 (segment (start -0.63 9.1) (end -0.63 13.9) (width 0.09) (layer B.Cu) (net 57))
 (segment (start -1.9 9.1) (end -1.9 13.9) (width 0.09) (layer B.Cu) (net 58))
 (segment (start -3.17 9.1) (end -3.17 13.9) (width 0.09) (layer B.Cu) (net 59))
 (segment (start -4.44 9.1) (end -4.44 13.9) (width 0.09) (layer B.Cu) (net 60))
 (segment (start -5.71 9.1) (end -5.71 13.9) (width 0.09) (layer B.Cu) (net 61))
 (segment (start 7.62 15) (end 7.62 8) (width 0.09) (layer F.Cu) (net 62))
 (segment (start 6.35 14.185002) (end 6.35 15) (width 0.09) (layer F.Cu) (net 63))
 (segment (start 6.35 8) (end 6.35 14.185002) (width 0.09) (layer F.Cu) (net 63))
 (segment (start 5.08 15) (end 5.08 8) (width 0.09) (layer F.Cu) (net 64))
 (segment (start 3.81 12.334998) (end 3.81 15) (width 0.09) (layer F.Cu) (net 65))
 (segment (start 3.81 8) (end 3.81 12.334998) (width 0.09) (layer F.Cu) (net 65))
 (segment (start 2.54 15) (end 2.54 8) (width 0.09) (layer F.Cu) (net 66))
 (segment (start 1.27 8) (end 1.27 15) (width 0.09) (layer F.Cu) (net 67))
 (segment (start 0 13.614998) (end 0 8) (width 0.09) (layer F.Cu) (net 68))
 (segment (start 0 15) (end 0 13.614998) (width 0.09) (layer F.Cu) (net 68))
 (segment (start -1.27 8) (end -1.27 15) (width 0.09) (layer F.Cu) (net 69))
 (segment (start -2.54 15) (end -2.54 8) (width 0.09) (layer F.Cu) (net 70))
 (segment (start -3.81 8) (end -3.81 15) (width 0.09) (layer F.Cu) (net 71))
 (segment (start -5.08 15) (end -5.08 8) (width 0.09) (layer F.Cu) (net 72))
 (segment (start -6.35 8) (end -6.35 15) (width 0.09) (layer F.Cu) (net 73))
 (segment (start -6.98 9.1) (end -6.98 13.9) (width 0.09) (layer B.Cu) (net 74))
 (segment (start -7.62 14.185002) (end -7.62 15) (width 0.09) (layer F.Cu) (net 75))
 (segment (start -7.62 8) (end -7.62 14.185002) (width 0.09) (layer F.Cu) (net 75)))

